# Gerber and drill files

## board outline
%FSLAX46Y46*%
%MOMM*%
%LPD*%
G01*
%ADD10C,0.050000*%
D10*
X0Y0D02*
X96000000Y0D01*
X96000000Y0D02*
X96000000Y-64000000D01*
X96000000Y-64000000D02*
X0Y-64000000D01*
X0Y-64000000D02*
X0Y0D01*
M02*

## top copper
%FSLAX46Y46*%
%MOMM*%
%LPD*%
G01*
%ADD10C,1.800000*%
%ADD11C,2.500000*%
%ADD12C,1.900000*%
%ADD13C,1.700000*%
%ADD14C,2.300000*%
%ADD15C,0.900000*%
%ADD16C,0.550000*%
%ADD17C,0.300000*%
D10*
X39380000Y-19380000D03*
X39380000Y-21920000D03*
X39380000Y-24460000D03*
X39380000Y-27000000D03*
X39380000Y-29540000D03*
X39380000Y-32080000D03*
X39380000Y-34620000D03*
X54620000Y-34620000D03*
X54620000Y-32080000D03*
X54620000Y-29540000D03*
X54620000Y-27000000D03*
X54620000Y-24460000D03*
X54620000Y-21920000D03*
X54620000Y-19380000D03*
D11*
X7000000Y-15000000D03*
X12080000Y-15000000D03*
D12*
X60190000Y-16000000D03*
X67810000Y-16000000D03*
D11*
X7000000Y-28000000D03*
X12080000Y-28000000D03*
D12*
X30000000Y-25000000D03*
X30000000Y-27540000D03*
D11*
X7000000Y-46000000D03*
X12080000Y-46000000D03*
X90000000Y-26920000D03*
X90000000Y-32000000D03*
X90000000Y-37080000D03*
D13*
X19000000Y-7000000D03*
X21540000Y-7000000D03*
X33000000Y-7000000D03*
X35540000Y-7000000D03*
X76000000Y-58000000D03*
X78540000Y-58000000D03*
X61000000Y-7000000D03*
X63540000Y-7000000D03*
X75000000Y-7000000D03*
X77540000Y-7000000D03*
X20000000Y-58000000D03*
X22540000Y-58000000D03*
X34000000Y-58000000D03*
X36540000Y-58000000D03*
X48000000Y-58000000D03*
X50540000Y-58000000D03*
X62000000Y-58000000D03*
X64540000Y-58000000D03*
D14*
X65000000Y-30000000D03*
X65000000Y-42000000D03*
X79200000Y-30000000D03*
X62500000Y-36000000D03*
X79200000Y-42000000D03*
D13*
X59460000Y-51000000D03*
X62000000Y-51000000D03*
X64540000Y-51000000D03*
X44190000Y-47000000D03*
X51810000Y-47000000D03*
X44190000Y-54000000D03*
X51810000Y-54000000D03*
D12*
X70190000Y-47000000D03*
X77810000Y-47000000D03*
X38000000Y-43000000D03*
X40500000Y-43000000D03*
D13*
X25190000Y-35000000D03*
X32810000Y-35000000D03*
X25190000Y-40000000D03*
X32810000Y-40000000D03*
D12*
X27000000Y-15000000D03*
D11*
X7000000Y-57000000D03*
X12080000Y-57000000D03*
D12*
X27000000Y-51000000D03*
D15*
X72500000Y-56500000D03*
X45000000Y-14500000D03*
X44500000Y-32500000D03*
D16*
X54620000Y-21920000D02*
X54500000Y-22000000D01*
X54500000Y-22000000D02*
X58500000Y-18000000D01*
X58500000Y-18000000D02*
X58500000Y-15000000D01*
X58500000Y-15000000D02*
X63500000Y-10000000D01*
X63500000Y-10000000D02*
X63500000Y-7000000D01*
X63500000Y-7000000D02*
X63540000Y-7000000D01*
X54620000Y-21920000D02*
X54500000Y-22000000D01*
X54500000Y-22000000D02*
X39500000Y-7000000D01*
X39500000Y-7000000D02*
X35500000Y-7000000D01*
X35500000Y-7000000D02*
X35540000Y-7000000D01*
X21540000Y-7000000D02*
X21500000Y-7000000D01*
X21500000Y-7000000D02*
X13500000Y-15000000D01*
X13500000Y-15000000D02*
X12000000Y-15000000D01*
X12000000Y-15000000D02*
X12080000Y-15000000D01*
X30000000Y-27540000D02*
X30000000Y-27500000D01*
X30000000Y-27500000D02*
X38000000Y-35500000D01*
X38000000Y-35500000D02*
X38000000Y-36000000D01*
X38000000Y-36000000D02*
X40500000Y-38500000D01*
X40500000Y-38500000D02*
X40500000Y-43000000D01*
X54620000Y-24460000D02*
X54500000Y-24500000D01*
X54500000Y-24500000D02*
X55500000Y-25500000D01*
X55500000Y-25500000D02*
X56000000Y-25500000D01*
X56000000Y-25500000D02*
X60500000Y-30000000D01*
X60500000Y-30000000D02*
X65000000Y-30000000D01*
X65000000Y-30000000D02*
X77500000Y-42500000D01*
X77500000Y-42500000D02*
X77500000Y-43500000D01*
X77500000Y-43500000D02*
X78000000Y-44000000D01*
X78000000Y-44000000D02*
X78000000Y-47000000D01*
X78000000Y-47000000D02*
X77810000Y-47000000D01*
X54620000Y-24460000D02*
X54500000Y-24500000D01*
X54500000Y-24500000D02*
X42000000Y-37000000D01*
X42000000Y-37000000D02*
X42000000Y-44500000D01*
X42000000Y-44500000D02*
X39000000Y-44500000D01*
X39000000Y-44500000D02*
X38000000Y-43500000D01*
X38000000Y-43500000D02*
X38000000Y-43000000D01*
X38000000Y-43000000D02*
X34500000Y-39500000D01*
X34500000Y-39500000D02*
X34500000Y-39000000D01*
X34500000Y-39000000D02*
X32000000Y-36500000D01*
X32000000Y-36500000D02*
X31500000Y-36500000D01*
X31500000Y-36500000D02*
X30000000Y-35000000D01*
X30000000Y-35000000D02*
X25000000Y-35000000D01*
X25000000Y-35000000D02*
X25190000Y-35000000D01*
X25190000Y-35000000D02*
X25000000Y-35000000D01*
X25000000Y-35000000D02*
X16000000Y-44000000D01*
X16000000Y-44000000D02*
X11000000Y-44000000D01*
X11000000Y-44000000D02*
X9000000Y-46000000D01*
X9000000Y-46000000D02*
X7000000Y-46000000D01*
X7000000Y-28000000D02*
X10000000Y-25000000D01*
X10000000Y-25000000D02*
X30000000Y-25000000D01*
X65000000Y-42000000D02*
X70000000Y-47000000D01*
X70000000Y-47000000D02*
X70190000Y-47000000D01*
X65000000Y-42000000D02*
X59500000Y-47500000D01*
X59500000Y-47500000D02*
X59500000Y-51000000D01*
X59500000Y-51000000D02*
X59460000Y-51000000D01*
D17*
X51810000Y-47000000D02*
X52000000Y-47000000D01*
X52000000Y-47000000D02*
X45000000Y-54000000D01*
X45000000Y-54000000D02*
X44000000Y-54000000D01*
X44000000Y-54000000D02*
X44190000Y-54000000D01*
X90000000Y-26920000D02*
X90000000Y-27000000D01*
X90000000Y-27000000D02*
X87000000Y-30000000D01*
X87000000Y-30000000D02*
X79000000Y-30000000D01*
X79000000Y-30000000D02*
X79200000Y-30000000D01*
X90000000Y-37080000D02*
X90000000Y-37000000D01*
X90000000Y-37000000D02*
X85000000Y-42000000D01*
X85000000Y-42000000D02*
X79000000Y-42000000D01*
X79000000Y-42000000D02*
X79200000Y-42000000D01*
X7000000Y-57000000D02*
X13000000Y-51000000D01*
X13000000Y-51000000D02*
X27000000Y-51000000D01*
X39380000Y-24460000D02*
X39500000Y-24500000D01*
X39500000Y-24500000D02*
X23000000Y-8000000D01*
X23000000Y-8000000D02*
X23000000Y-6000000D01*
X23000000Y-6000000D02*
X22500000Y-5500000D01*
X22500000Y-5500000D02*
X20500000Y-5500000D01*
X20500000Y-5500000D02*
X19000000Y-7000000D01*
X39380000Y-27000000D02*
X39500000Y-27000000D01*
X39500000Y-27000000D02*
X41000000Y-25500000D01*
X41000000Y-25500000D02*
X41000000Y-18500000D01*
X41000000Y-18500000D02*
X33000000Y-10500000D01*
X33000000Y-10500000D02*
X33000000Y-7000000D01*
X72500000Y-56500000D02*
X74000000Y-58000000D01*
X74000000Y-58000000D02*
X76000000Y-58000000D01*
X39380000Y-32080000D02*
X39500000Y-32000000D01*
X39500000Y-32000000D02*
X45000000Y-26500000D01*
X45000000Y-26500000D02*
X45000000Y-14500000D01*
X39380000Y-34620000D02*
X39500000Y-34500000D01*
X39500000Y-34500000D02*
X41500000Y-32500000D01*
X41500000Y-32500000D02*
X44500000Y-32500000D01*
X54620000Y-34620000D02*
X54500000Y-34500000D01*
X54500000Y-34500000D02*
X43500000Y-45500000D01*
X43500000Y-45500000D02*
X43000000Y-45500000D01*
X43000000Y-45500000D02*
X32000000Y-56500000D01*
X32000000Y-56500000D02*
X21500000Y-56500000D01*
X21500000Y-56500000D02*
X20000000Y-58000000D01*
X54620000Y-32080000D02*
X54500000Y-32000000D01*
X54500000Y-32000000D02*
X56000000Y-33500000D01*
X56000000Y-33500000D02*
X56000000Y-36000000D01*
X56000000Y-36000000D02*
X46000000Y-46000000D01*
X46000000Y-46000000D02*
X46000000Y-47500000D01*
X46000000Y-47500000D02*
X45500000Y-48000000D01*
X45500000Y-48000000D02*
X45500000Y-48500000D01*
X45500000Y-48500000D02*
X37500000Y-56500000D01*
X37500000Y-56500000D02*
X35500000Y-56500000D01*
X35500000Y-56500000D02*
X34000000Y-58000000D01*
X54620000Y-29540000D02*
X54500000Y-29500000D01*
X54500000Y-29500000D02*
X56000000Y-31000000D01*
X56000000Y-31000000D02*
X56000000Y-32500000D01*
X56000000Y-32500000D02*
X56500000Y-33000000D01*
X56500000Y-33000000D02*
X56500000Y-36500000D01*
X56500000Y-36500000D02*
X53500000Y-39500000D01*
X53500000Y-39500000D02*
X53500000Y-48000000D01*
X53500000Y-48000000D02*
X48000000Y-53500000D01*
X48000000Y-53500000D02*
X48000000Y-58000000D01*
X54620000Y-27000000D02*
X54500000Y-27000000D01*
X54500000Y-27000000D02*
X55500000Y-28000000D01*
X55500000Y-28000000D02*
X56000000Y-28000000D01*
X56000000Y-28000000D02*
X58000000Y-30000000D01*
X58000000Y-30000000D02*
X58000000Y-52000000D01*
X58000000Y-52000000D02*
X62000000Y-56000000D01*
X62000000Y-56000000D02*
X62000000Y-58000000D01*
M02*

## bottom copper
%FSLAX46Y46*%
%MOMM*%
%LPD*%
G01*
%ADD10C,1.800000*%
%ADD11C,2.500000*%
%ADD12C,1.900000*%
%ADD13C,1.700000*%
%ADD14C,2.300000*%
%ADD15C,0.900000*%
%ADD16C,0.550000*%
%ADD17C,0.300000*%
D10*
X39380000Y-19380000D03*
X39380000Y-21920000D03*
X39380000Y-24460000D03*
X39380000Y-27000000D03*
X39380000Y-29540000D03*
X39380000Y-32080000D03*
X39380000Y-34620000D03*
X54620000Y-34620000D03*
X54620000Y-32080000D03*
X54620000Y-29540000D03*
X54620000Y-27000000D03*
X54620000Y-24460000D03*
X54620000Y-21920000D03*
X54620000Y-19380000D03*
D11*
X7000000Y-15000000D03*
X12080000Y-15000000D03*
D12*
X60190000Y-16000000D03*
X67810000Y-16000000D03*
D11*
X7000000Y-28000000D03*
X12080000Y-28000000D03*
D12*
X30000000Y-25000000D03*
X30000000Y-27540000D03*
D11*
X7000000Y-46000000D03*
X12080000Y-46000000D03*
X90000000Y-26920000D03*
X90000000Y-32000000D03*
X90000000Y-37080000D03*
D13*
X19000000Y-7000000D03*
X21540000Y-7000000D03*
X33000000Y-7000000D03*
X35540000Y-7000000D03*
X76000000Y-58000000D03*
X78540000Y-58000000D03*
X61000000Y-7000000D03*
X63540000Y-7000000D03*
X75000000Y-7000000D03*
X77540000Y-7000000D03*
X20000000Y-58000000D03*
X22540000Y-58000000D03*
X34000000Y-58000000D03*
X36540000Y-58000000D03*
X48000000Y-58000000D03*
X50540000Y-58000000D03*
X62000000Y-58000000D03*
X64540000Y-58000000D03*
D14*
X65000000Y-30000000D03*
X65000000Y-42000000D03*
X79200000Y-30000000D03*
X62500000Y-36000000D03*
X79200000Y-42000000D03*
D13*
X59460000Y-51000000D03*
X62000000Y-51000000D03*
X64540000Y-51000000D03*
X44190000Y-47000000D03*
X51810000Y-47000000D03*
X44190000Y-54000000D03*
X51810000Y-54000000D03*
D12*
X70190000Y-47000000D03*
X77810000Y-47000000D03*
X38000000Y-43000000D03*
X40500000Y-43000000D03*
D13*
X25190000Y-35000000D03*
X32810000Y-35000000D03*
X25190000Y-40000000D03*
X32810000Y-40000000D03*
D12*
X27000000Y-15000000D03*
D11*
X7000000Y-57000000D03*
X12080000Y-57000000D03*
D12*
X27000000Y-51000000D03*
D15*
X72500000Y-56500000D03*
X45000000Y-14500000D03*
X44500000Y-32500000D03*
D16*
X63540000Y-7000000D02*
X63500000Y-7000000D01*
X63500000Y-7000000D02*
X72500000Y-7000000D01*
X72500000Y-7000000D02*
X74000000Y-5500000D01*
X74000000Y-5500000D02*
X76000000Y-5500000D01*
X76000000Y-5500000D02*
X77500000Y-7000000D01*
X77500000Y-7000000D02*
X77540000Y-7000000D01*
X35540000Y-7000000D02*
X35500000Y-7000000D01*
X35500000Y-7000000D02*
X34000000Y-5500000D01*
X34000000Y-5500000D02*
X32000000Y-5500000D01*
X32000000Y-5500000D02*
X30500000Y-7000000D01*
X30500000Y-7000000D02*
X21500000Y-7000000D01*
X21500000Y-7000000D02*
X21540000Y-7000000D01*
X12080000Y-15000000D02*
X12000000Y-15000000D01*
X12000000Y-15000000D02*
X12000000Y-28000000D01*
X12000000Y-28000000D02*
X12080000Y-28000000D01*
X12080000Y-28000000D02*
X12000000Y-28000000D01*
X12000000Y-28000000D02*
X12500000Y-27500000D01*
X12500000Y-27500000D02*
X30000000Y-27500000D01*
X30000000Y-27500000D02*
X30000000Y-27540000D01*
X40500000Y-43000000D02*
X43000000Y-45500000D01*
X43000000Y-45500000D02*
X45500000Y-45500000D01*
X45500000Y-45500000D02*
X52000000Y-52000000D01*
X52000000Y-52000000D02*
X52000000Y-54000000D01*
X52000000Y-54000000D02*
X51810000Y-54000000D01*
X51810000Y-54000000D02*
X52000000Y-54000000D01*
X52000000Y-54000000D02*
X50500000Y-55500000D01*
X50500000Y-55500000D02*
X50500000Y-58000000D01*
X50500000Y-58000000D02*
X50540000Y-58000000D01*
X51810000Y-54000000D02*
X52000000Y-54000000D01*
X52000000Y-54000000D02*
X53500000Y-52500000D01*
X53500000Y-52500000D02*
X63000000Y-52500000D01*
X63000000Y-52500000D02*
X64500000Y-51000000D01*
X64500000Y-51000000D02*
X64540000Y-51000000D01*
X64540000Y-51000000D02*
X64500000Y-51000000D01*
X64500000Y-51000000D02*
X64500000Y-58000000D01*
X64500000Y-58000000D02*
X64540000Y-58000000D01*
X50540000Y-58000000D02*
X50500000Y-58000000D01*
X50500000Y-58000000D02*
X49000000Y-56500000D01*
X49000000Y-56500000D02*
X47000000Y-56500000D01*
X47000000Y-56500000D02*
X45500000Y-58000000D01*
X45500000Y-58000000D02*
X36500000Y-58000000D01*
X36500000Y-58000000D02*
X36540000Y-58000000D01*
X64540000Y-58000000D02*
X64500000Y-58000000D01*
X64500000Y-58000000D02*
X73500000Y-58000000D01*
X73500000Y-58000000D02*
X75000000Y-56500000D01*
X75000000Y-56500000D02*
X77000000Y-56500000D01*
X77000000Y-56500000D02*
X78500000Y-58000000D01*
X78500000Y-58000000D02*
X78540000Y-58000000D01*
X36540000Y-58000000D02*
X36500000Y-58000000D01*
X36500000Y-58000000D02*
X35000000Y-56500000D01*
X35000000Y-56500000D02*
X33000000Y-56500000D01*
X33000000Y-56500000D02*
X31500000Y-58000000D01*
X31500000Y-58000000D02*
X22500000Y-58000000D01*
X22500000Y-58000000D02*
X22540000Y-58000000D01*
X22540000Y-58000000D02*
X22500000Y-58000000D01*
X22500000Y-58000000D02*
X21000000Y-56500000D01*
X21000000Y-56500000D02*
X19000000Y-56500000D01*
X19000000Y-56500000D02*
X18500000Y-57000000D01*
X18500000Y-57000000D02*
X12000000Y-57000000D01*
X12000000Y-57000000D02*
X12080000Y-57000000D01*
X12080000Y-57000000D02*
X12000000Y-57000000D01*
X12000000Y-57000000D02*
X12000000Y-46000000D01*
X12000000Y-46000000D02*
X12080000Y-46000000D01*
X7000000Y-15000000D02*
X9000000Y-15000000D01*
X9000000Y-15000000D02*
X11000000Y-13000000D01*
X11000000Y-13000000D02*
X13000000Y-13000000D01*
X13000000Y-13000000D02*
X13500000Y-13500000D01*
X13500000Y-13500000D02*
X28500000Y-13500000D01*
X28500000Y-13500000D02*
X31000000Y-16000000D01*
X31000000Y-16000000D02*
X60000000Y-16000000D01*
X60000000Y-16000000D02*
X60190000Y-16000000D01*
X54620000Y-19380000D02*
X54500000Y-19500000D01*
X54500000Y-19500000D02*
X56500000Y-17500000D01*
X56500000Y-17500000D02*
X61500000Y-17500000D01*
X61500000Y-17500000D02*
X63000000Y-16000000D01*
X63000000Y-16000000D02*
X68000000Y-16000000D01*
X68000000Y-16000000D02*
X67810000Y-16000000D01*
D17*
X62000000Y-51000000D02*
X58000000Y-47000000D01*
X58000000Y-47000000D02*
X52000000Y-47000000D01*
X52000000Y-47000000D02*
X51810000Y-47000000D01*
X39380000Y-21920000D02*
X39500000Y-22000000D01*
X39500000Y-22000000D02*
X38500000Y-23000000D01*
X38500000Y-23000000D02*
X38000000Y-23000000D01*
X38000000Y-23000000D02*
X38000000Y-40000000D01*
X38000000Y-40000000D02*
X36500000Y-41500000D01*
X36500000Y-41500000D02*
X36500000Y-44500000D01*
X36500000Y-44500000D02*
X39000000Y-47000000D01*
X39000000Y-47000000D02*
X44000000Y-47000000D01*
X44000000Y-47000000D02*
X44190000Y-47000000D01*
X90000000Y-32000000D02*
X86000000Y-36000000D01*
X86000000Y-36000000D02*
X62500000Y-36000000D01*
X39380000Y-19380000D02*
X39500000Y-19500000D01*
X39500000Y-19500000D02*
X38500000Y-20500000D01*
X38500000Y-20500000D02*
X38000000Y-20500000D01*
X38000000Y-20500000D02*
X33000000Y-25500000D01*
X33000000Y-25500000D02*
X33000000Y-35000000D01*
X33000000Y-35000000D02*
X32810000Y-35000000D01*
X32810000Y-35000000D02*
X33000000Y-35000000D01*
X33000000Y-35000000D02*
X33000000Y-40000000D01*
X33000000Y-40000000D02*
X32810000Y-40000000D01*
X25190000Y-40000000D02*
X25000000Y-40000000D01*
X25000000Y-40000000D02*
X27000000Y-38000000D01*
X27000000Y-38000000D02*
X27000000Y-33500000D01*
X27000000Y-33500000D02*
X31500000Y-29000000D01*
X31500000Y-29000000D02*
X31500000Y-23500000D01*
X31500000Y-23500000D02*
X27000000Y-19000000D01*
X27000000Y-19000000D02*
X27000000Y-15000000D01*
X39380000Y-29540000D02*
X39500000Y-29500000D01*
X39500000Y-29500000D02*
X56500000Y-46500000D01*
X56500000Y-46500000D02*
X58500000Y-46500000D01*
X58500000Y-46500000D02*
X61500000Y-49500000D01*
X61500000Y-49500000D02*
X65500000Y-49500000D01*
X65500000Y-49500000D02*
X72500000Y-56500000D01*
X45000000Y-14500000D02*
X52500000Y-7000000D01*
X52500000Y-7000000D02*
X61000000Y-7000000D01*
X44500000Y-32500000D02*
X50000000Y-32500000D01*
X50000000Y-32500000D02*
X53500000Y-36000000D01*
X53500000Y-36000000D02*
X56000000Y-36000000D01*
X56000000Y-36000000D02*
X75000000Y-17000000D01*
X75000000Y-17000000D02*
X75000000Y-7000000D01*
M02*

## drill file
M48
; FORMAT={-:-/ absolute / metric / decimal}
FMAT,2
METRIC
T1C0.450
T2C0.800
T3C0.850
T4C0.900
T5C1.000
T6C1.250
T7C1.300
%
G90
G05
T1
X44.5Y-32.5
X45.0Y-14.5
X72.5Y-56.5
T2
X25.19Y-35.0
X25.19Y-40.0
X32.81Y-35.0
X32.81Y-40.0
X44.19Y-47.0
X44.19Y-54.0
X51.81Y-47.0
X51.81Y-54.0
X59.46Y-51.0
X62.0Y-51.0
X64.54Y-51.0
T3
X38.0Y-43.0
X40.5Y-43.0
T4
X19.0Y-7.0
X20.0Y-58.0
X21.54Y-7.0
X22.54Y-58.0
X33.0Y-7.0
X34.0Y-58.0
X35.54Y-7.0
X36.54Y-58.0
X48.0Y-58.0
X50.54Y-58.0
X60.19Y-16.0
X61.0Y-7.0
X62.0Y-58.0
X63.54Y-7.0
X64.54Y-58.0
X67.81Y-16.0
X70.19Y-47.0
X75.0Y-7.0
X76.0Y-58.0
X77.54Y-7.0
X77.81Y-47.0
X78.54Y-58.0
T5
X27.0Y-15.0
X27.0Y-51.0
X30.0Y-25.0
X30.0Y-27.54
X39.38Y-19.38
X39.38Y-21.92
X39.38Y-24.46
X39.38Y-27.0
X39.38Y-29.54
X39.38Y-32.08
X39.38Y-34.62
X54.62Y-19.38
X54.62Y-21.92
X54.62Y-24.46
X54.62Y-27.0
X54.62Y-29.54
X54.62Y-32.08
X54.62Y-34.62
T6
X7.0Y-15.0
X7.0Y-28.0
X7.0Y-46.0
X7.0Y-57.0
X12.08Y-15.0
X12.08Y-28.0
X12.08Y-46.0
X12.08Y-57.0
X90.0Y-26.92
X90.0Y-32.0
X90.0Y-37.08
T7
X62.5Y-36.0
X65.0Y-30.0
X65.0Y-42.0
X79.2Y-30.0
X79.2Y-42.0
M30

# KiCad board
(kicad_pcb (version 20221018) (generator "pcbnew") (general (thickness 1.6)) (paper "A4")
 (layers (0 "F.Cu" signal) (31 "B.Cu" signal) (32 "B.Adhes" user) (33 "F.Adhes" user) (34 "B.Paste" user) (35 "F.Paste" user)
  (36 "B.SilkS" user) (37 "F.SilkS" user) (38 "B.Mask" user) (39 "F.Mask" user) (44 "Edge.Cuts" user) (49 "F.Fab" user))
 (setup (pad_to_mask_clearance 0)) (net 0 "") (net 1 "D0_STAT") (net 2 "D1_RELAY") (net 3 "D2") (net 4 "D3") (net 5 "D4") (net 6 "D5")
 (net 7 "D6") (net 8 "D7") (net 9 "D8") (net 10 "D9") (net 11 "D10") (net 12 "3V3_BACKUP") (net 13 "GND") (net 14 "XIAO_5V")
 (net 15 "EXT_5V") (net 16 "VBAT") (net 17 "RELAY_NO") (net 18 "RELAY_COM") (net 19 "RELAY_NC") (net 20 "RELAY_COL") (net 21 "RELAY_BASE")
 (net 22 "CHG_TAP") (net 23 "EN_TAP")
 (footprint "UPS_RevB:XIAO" (layer "F.Cu") (at 47 27)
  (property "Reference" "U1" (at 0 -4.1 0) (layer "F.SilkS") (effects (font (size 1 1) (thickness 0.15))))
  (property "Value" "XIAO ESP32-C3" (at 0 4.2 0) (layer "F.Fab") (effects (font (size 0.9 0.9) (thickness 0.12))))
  (pad "1" thru_hole circle (at -7.62 -7.62) (size 1.8 1.8) (drill 1) (layers "*.Cu" "*.Mask") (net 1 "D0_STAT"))
  (pad "2" thru_hole circle (at -7.62 -5.08) (size 1.8 1.8) (drill 1) (layers "*.Cu" "*.Mask") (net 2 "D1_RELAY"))
  (pad "3" thru_hole circle (at -7.62 -2.54) (size 1.8 1.8) (drill 1) (layers "*.Cu" "*.Mask") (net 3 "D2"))
  (pad "4" thru_hole circle (at -7.62 0) (size 1.8 1.8) (drill 1) (layers "*.Cu" "*.Mask") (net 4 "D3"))
  (pad "5" thru_hole circle (at -7.62 2.54) (size 1.8 1.8) (drill 1) (layers "*.Cu" "*.Mask") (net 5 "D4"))
  (pad "6" thru_hole circle (at -7.62 5.08) (size 1.8 1.8) (drill 1) (layers "*.Cu" "*.Mask") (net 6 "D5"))
  (pad "7" thru_hole circle (at -7.62 7.62) (size 1.8 1.8) (drill 1) (layers "*.Cu" "*.Mask") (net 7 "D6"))
  (pad "8" thru_hole circle (at 7.62 7.62) (size 1.8 1.8) (drill 1) (layers "*.Cu" "*.Mask") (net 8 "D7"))
  (pad "9" thru_hole circle (at 7.62 5.08) (size 1.8 1.8) (drill 1) (layers "*.Cu" "*.Mask") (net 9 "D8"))
  (pad "10" thru_hole circle (at 7.62 2.54) (size 1.8 1.8) (drill 1) (layers "*.Cu" "*.Mask") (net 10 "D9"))
  (pad "11" thru_hole circle (at 7.62 0) (size 1.8 1.8) (drill 1) (layers "*.Cu" "*.Mask") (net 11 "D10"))
  (pad "12" thru_hole circle (at 7.62 -2.54) (size 1.8 1.8) (drill 1) (layers "*.Cu" "*.Mask") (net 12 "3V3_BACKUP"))
  (pad "13" thru_hole circle (at 7.62 -5.08) (size 1.8 1.8) (drill 1) (layers "*.Cu" "*.Mask") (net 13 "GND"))
  (pad "14" thru_hole circle (at 7.62 -7.62) (size 1.8 1.8) (drill 1) (layers "*.Cu" "*.Mask") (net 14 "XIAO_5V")))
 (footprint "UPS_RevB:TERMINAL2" (layer "F.Cu") (at 7 15)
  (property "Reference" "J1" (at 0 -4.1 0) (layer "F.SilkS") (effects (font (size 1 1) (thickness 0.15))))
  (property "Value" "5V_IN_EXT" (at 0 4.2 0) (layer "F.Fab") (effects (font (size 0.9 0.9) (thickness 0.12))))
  (pad "1" thru_hole circle (at 0 0) (size 2.5 2.5) (drill 1.25) (layers "*.Cu" "*.Mask") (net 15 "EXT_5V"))
  (pad "2" thru_hole circle (at 5.08 0) (size 2.5 2.5) (drill 1.25) (layers "*.Cu" "*.Mask") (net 13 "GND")))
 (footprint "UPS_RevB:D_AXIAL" (layer "F.Cu") (at 64 16)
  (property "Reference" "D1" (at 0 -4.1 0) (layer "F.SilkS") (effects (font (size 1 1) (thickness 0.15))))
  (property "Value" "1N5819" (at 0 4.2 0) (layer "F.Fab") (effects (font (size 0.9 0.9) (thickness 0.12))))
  (pad "1" thru_hole circle (at -3.81 0) (size 1.9 1.9) (drill 0.9) (layers "*.Cu" "*.Mask") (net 15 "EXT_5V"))
  (pad "2" thru_hole circle (at 3.81 0) (size 1.9 1.9) (drill 0.9) (layers "*.Cu" "*.Mask") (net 14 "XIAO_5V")))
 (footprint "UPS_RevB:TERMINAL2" (layer "F.Cu") (at 7 28)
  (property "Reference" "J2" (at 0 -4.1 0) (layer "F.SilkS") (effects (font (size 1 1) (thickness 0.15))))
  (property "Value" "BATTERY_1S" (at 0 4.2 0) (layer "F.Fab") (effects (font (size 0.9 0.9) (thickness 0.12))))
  (pad "1" thru_hole circle (at 0 0) (size 2.5 2.5) (drill 1.25) (layers "*.Cu" "*.Mask") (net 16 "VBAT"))
  (pad "2" thru_hole circle (at 5.08 0) (size 2.5 2.5) (drill 1.25) (layers "*.Cu" "*.Mask") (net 13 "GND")))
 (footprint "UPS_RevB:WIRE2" (layer "F.Cu") (at 30 25)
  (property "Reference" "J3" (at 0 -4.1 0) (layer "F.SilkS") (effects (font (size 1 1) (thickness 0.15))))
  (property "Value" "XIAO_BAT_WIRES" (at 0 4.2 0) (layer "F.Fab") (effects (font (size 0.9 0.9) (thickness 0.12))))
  (pad "1" thru_hole circle (at 0 0) (size 1.9 1.9) (drill 1) (layers "*.Cu" "*.Mask") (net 16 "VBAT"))
  (pad "2" thru_hole circle (at 0 2.54) (size 1.9 1.9) (drill 1) (layers "*.Cu" "*.Mask") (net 13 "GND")))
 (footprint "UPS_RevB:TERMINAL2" (layer "F.Cu") (at 7 46)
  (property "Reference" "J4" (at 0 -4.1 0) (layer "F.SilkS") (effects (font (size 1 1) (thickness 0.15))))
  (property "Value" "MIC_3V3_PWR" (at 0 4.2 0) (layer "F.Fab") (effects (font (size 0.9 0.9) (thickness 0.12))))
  (pad "1" thru_hole circle (at 0 0) (size 2.5 2.5) (drill 1.25) (layers "*.Cu" "*.Mask") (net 12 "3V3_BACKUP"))
  (pad "2" thru_hole circle (at 5.08 0) (size 2.5 2.5) (drill 1.25) (layers "*.Cu" "*.Mask") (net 13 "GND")))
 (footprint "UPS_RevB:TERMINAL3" (layer "F.Cu") (at 90 32)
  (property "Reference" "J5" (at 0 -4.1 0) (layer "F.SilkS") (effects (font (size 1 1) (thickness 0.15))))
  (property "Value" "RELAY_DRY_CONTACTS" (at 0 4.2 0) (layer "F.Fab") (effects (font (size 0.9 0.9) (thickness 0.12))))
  (pad "1" thru_hole circle (at 0 -5.08) (size 2.5 2.5) (drill 1.25) (layers "*.Cu" "*.Mask") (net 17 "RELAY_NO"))
  (pad "2" thru_hole circle (at 0 0) (size 2.5 2.5) (drill 1.25) (layers "*.Cu" "*.Mask") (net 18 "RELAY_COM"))
  (pad "3" thru_hole circle (at 0 5.08) (size 2.5 2.5) (drill 1.25) (layers "*.Cu" "*.Mask") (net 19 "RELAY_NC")))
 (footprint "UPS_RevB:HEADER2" (layer "F.Cu") (at 19 7)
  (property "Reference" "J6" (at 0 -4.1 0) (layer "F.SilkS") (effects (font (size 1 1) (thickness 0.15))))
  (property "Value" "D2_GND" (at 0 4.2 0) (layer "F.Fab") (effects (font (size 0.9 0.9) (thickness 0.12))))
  (pad "1" thru_hole circle (at 0 0) (size 1.7 1.7) (drill 0.9) (layers "*.Cu" "*.Mask") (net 3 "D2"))
  (pad "2" thru_hole circle (at 2.54 0) (size 1.7 1.7) (drill 0.9) (layers "*.Cu" "*.Mask") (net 13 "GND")))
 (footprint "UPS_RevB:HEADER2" (layer "F.Cu") (at 33 7)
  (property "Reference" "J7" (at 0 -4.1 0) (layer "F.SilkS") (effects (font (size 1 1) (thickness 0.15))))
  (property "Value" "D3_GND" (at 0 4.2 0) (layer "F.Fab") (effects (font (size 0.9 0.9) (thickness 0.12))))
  (pad "1" thru_hole circle (at 0 0) (size 1.7 1.7) (drill 0.9) (layers "*.Cu" "*.Mask") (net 4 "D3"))
  (pad "2" thru_hole circle (at 2.54 0) (size 1.7 1.7) (drill 0.9) (layers "*.Cu" "*.Mask") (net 13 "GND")))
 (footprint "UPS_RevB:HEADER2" (layer "F.Cu") (at 76 58)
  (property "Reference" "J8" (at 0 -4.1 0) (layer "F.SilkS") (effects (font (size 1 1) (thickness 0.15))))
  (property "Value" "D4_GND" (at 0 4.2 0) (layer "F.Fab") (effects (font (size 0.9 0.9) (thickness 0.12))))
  (pad "1" thru_hole circle (at 0 0) (size 1.7 1.7) (drill 0.9) (layers "*.Cu" "*.Mask") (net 5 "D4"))
  (pad "2" thru_hole circle (at 2.54 0) (size 1.7 1.7) (drill 0.9) (layers "*.Cu" "*.Mask") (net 13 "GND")))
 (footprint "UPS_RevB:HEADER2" (layer "F.Cu") (at 61 7)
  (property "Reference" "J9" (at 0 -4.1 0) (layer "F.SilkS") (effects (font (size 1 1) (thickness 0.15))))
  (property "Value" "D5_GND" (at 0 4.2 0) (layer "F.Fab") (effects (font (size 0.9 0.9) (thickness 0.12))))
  (pad "1" thru_hole circle (at 0 0) (size 1.7 1.7) (drill 0.9) (layers "*.Cu" "*.Mask") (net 6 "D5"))
  (pad "2" thru_hole circle (at 2.54 0) (size 1.7 1.7) (drill 0.9) (layers "*.Cu" "*.Mask") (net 13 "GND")))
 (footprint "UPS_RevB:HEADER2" (layer "F.Cu") (at 75 7)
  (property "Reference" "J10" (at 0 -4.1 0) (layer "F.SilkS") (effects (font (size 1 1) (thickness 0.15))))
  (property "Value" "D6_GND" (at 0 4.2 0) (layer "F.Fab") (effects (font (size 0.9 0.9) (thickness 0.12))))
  (pad "1" thru_hole circle (at 0 0) (size 1.7 1.7) (drill 0.9) (layers "*.Cu" "*.Mask") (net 7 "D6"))
  (pad "2" thru_hole circle (at 2.54 0) (size 1.7 1.7) (drill 0.9) (layers "*.Cu" "*.Mask") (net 13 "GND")))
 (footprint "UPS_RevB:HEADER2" (layer "F.Cu") (at 20 58)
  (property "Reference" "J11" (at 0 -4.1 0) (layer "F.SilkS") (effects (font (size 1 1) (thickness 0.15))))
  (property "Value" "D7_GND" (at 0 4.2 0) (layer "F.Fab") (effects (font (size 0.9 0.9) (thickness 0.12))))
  (pad "1" thru_hole circle (at 0 0) (size 1.7 1.7) (drill 0.9) (layers "*.Cu" "*.Mask") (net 8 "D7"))
  (pad "2" thru_hole circle (at 2.54 0) (size 1.7 1.7) (drill 0.9) (layers "*.Cu" "*.Mask") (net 13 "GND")))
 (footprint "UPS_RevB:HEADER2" (layer "F.Cu") (at 34 58)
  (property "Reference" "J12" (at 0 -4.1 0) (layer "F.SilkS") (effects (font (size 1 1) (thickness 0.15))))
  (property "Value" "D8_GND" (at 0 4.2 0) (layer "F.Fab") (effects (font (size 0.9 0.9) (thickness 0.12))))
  (pad "1" thru_hole circle (at 0 0) (size 1.7 1.7) (drill 0.9) (layers "*.Cu" "*.Mask") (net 9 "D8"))
  (pad "2" thru_hole circle (at 2.54 0) (size 1.7 1.7) (drill 0.9) (layers "*.Cu" "*.Mask") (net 13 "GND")))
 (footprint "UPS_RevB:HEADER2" (layer "F.Cu") (at 48 58)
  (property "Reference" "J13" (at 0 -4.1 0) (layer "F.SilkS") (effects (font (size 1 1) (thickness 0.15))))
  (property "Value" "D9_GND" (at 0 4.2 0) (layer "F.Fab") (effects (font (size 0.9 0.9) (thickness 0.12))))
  (pad "1" thru_hole circle (at 0 0) (size 1.7 1.7) (drill 0.9) (layers "*.Cu" "*.Mask") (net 10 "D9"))
  (pad "2" thru_hole circle (at 2.54 0) (size 1.7 1.7) (drill 0.9) (layers "*.Cu" "*.Mask") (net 13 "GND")))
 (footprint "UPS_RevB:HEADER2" (layer "F.Cu") (at 62 58)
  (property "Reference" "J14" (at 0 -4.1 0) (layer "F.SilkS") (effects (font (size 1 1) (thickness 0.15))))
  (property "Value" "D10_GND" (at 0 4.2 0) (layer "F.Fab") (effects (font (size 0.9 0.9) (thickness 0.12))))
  (pad "1" thru_hole circle (at 0 0) (size 1.7 1.7) (drill 0.9) (layers "*.Cu" "*.Mask") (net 11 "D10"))
  (pad "2" thru_hole circle (at 2.54 0) (size 1.7 1.7) (drill 0.9) (layers "*.Cu" "*.Mask") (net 13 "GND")))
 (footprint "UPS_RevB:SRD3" (layer "F.Cu") (at 65 30)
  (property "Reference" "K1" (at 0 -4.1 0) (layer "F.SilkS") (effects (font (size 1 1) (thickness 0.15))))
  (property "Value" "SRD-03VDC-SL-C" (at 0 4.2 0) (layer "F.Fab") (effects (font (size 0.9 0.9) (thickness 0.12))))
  (pad "1" thru_hole circle (at 0 0) (size 2.3 2.3) (drill 1.3) (layers "*.Cu" "*.Mask") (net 12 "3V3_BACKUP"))
  (pad "2" thru_hole circle (at 0 12) (size 2.3 2.3) (drill 1.3) (layers "*.Cu" "*.Mask") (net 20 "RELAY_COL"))
  (pad "3" thru_hole circle (at 14.2 0) (size 2.3 2.3) (drill 1.3) (layers "*.Cu" "*.Mask") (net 17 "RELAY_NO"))
  (pad "4" thru_hole circle (at -2.5 6) (size 2.3 2.3) (drill 1.3) (layers "*.Cu" "*.Mask") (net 18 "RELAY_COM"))
  (pad "5" thru_hole circle (at 14.2 12) (size 2.3 2.3) (drill 1.3) (layers "*.Cu" "*.Mask") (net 19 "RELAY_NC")))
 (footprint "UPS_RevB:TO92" (layer "F.Cu") (at 62 51)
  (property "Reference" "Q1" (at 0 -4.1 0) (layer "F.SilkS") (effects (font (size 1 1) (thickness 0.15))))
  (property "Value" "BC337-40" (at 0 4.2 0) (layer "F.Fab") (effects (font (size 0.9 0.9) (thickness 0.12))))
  (pad "1" thru_hole circle (at -2.54 0) (size 1.7 1.7) (drill 0.8) (layers "*.Cu" "*.Mask") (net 20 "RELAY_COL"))
  (pad "2" thru_hole circle (at 0 0) (size 1.7 1.7) (drill 0.8) (layers "*.Cu" "*.Mask") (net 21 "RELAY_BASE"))
  (pad "3" thru_hole circle (at 2.54 0) (size 1.7 1.7) (drill 0.8) (layers "*.Cu" "*.Mask") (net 13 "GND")))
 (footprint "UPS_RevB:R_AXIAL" (layer "F.Cu") (at 48 47)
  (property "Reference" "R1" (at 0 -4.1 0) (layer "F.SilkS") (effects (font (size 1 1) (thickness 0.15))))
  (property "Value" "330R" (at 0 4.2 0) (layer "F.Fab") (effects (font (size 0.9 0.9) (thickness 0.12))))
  (pad "1" thru_hole circle (at -3.81 0) (size 1.7 1.7) (drill 0.8) (layers "*.Cu" "*.Mask") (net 2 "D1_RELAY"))
  (pad "2" thru_hole circle (at 3.81 0) (size 1.7 1.7) (drill 0.8) (layers "*.Cu" "*.Mask") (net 21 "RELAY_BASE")))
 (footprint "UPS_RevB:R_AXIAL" (layer "F.Cu") (at 48 54)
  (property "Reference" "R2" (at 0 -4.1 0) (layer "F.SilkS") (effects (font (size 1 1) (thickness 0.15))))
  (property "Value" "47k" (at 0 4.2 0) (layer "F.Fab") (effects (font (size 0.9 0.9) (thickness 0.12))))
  (pad "1" thru_hole circle (at -3.81 0) (size 1.7 1.7) (drill 0.8) (layers "*.Cu" "*.Mask") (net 21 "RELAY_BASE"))
  (pad "2" thru_hole circle (at 3.81 0) (size 1.7 1.7) (drill 0.8) (layers "*.Cu" "*.Mask") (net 13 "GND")))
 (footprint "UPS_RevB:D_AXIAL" (layer "F.Cu") (at 74 47)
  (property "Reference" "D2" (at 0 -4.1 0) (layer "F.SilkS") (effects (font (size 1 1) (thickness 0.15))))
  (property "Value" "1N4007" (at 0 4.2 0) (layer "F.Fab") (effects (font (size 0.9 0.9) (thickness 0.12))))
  (pad "1" thru_hole circle (at -3.81 0) (size 1.9 1.9) (drill 0.9) (layers "*.Cu" "*.Mask") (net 20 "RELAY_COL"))
  (pad "2" thru_hole circle (at 3.81 0) (size 1.9 1.9) (drill 0.9) (layers "*.Cu" "*.Mask") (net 12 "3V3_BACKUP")))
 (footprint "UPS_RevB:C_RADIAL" (layer "F.Cu") (at 38 43)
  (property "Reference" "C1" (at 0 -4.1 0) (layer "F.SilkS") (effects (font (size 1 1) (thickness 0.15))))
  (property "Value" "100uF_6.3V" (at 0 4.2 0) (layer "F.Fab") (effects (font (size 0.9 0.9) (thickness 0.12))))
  (pad "1" thru_hole circle (at 0 0) (size 1.9 1.9) (drill 0.85) (layers "*.Cu" "*.Mask") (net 12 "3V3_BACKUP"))
  (pad "2" thru_hole circle (at 2.5 0) (size 1.9 1.9) (drill 0.85) (layers "*.Cu" "*.Mask") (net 13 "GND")))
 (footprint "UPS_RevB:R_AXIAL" (layer "F.Cu") (at 29 35)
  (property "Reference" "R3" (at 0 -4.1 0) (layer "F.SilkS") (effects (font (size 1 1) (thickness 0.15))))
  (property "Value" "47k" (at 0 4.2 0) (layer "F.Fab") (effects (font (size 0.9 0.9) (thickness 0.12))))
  (pad "1" thru_hole circle (at -3.81 0) (size 1.7 1.7) (drill 0.8) (layers "*.Cu" "*.Mask") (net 12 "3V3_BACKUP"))
  (pad "2" thru_hole circle (at 3.81 0) (size 1.7 1.7) (drill 0.8) (layers "*.Cu" "*.Mask") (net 1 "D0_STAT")))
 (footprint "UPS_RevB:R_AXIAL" (layer "F.Cu") (at 29 40)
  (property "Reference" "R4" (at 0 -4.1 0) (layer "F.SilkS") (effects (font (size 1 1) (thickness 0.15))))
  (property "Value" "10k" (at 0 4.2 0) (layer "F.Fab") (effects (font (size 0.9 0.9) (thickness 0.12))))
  (pad "1" thru_hole circle (at -3.81 0) (size 1.7 1.7) (drill 0.8) (layers "*.Cu" "*.Mask") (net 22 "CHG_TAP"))
  (pad "2" thru_hole circle (at 3.81 0) (size 1.7 1.7) (drill 0.8) (layers "*.Cu" "*.Mask") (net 1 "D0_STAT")))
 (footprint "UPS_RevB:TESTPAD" (layer "F.Cu") (at 27 15)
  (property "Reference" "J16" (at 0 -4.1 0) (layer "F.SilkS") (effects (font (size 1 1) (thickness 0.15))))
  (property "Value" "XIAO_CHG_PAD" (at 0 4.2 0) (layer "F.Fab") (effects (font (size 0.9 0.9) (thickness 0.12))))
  (pad "1" thru_hole circle (at 0 0) (size 1.9 1.9) (drill 1) (layers "*.Cu" "*.Mask") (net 22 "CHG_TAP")))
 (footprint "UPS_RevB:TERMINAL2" (layer "F.Cu") (at 7 57)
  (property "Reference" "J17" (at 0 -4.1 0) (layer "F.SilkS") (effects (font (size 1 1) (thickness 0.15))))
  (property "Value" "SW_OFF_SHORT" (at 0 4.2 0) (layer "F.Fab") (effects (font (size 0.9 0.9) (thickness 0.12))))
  (pad "1" thru_hole circle (at 0 0) (size 2.5 2.5) (drill 1.25) (layers "*.Cu" "*.Mask") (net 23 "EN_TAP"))
  (pad "2" thru_hole circle (at 5.08 0) (size 2.5 2.5) (drill 1.25) (layers "*.Cu" "*.Mask") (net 13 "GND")))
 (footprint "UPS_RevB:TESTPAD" (layer "F.Cu") (at 27 51)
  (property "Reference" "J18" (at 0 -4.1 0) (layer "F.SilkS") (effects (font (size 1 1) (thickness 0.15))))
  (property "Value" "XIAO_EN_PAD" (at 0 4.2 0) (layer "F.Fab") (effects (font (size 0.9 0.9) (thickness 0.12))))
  (pad "1" thru_hole circle (at 0 0) (size 1.9 1.9) (drill 1) (layers "*.Cu" "*.Mask") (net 23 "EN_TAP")))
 (gr_line (start 0 0) (end 96 0) (stroke (width 0.05) (type default)) (layer "Edge.Cuts"))
 (gr_line (start 96 0) (end 96 64) (stroke (width 0.05) (type default)) (layer "Edge.Cuts"))
 (gr_line (start 96 64) (end 0 64) (stroke (width 0.05) (type default)) (layer "Edge.Cuts"))
 (gr_line (start 0 64) (end 0 0) (stroke (width 0.05) (type default)) (layer "Edge.Cuts"))
 (segment (start 54.62 21.92) (end 54.5 22) (width 0.55) (layer "F.Cu") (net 13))
 (segment (start 54.5 22) (end 58.5 18) (width 0.55) (layer "F.Cu") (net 13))
 (segment (start 58.5 18) (end 58.5 15) (width 0.55) (layer "F.Cu") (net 13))
 (segment (start 58.5 15) (end 63.5 10) (width 0.55) (layer "F.Cu") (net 13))
 (segment (start 63.5 10) (end 63.5 7) (width 0.55) (layer "F.Cu") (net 13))
 (segment (start 63.5 7) (end 63.54 7) (width 0.55) (layer "F.Cu") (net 13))
 (segment (start 63.54 7) (end 63.5 7) (width 0.55) (layer "B.Cu") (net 13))
 (segment (start 63.5 7) (end 72.5 7) (width 0.55) (layer "B.Cu") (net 13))
 (segment (start 72.5 7) (end 74 5.5) (width 0.55) (layer "B.Cu") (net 13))
 (segment (start 74 5.5) (end 76 5.5) (width 0.55) (layer "B.Cu") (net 13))
 (segment (start 76 5.5) (end 77.5 7) (width 0.55) (layer "B.Cu") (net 13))
 (segment (start 77.5 7) (end 77.54 7) (width 0.55) (layer "B.Cu") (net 13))
 (segment (start 54.62 21.92) (end 54.5 22) (width 0.55) (layer "F.Cu") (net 13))
 (segment (start 54.5 22) (end 39.5 7) (width 0.55) (layer "F.Cu") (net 13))
 (segment (start 39.5 7) (end 35.5 7) (width 0.55) (layer "F.Cu") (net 13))
 (segment (start 35.5 7) (end 35.54 7) (width 0.55) (layer "F.Cu") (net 13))
 (segment (start 35.54 7) (end 35.5 7) (width 0.55) (layer "B.Cu") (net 13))
 (segment (start 35.5 7) (end 34 5.5) (width 0.55) (layer "B.Cu") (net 13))
 (segment (start 34 5.5) (end 32 5.5) (width 0.55) (layer "B.Cu") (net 13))
 (segment (start 32 5.5) (end 30.5 7) (width 0.55) (layer "B.Cu") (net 13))
 (segment (start 30.5 7) (end 21.5 7) (width 0.55) (layer "B.Cu") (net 13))
 (segment (start 21.5 7) (end 21.54 7) (width 0.55) (layer "B.Cu") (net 13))
 (segment (start 21.54 7) (end 21.5 7) (width 0.55) (layer "F.Cu") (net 13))
 (segment (start 21.5 7) (end 13.5 15) (width 0.55) (layer "F.Cu") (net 13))
 (segment (start 13.5 15) (end 12 15) (width 0.55) (layer "F.Cu") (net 13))
 (segment (start 12 15) (end 12.08 15) (width 0.55) (layer "F.Cu") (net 13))
 (segment (start 12.08 15) (end 12 15) (width 0.55) (layer "B.Cu") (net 13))
 (segment (start 12 15) (end 12 28) (width 0.55) (layer "B.Cu") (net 13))
 (segment (start 12 28) (end 12.08 28) (width 0.55) (layer "B.Cu") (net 13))
 (segment (start 12.08 28) (end 12 28) (width 0.55) (layer "B.Cu") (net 13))
 (segment (start 12 28) (end 12.5 27.5) (width 0.55) (layer "B.Cu") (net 13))
 (segment (start 12.5 27.5) (end 30 27.5) (width 0.55) (layer "B.Cu") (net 13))
 (segment (start 30 27.5) (end 30 27.54) (width 0.55) (layer "B.Cu") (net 13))
 (segment (start 30 27.54) (end 30 27.5) (width 0.55) (layer "F.Cu") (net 13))
 (segment (start 30 27.5) (end 38 35.5) (width 0.55) (layer "F.Cu") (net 13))
 (segment (start 38 35.5) (end 38 36) (width 0.55) (layer "F.Cu") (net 13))
 (segment (start 38 36) (end 40.5 38.5) (width 0.55) (layer "F.Cu") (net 13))
 (segment (start 40.5 38.5) (end 40.5 43) (width 0.55) (layer "F.Cu") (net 13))
 (segment (start 40.5 43) (end 43 45.5) (width 0.55) (layer "B.Cu") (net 13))
 (segment (start 43 45.5) (end 45.5 45.5) (width 0.55) (layer "B.Cu") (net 13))
 (segment (start 45.5 45.5) (end 52 52) (width 0.55) (layer "B.Cu") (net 13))
 (segment (start 52 52) (end 52 54) (width 0.55) (layer "B.Cu") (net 13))
 (segment (start 52 54) (end 51.81 54) (width 0.55) (layer "B.Cu") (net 13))
 (segment (start 51.81 54) (end 52 54) (width 0.55) (layer "B.Cu") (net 13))
 (segment (start 52 54) (end 50.5 55.5) (width 0.55) (layer "B.Cu") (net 13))
 (segment (start 50.5 55.5) (end 50.5 58) (width 0.55) (layer "B.Cu") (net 13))
 (segment (start 50.5 58) (end 50.54 58) (width 0.55) (layer "B.Cu") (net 13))
 (segment (start 51.81 54) (end 52 54) (width 0.55) (layer "B.Cu") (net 13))
 (segment (start 52 54) (end 53.5 52.5) (width 0.55) (layer "B.Cu") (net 13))
 (segment (start 53.5 52.5) (end 63 52.5) (width 0.55) (layer "B.Cu") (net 13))
 (segment (start 63 52.5) (end 64.5 51) (width 0.55) (layer "B.Cu") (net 13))
 (segment (start 64.5 51) (end 64.54 51) (width 0.55) (layer "B.Cu") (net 13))
 (segment (start 64.54 51) (end 64.5 51) (width 0.55) (layer "B.Cu") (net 13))
 (segment (start 64.5 51) (end 64.5 58) (width 0.55) (layer "B.Cu") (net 13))
 (segment (start 64.5 58) (end 64.54 58) (width 0.55) (layer "B.Cu") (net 13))
 (segment (start 50.54 58) (end 50.5 58) (width 0.55) (layer "B.Cu") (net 13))
 (segment (start 50.5 58) (end 49 56.5) (width 0.55) (layer "B.Cu") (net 13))
 (segment (start 49 56.5) (end 47 56.5) (width 0.55) (layer "B.Cu") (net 13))
 (segment (start 47 56.5) (end 45.5 58) (width 0.55) (layer "B.Cu") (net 13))
 (segment (start 45.5 58) (end 36.5 58) (width 0.55) (layer "B.Cu") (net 13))
 (segment (start 36.5 58) (end 36.54 58) (width 0.55) (layer "B.Cu") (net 13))
 (segment (start 64.54 58) (end 64.5 58) (width 0.55) (layer "B.Cu") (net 13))
 (segment (start 64.5 58) (end 73.5 58) (width 0.55) (layer "B.Cu") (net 13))
 (segment (start 73.5 58) (end 75 56.5) (width 0.55) (layer "B.Cu") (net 13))
 (segment (start 75 56.5) (end 77 56.5) (width 0.55) (layer "B.Cu") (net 13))
 (segment (start 77 56.5) (end 78.5 58) (width 0.55) (layer "B.Cu") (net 13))
 (segment (start 78.5 58) (end 78.54 58) (width 0.55) (layer "B.Cu") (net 13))
 (segment (start 36.54 58) (end 36.5 58) (width 0.55) (layer "B.Cu") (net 13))
 (segment (start 36.5 58) (end 35 56.5) (width 0.55) (layer "B.Cu") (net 13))
 (segment (start 35 56.5) (end 33 56.5) (width 0.55) (layer "B.Cu") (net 13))
 (segment (start 33 56.5) (end 31.5 58) (width 0.55) (layer "B.Cu") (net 13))
 (segment (start 31.5 58) (end 22.5 58) (width 0.55) (layer "B.Cu") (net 13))
 (segment (start 22.5 58) (end 22.54 58) (width 0.55) (layer "B.Cu") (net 13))
 (segment (start 22.54 58) (end 22.5 58) (width 0.55) (layer "B.Cu") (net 13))
 (segment (start 22.5 58) (end 21 56.5) (width 0.55) (layer "B.Cu") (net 13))
 (segment (start 21 56.5) (end 19 56.5) (width 0.55) (layer "B.Cu") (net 13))
 (segment (start 19 56.5) (end 18.5 57) (width 0.55) (layer "B.Cu") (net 13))
 (segment (start 18.5 57) (end 12 57) (width 0.55) (layer "B.Cu") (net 13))
 (segment (start 12 57) (end 12.08 57) (width 0.55) (layer "B.Cu") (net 13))
 (segment (start 12.08 57) (end 12 57) (width 0.55) (layer "B.Cu") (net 13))
 (segment (start 12 57) (end 12 46) (width 0.55) (layer "B.Cu") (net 13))
 (segment (start 12 46) (end 12.08 46) (width 0.55) (layer "B.Cu") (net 13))
 (segment (start 54.62 24.46) (end 54.5 24.5) (width 0.55) (layer "F.Cu") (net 12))
 (segment (start 54.5 24.5) (end 55.5 25.5) (width 0.55) (layer "F.Cu") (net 12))
 (segment (start 55.5 25.5) (end 56 25.5) (width 0.55) (layer "F.Cu") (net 12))
 (segment (start 56 25.5) (end 60.5 30) (width 0.55) (layer "F.Cu") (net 12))
 (segment (start 60.5 30) (end 65 30) (width 0.55) (layer "F.Cu") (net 12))
 (segment (start 65 30) (end 77.5 42.5) (width 0.55) (layer "F.Cu") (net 12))
 (segment (start 77.5 42.5) (end 77.5 43.5) (width 0.55) (layer "F.Cu") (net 12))
 (segment (start 77.5 43.5) (end 78 44) (width 0.55) (layer "F.Cu") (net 12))
 (segment (start 78 44) (end 78 47) (width 0.55) (layer "F.Cu") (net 12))
 (segment (start 78 47) (end 77.81 47) (width 0.55) (layer "F.Cu") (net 12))
 (segment (start 54.62 24.46) (end 54.5 24.5) (width 0.55) (layer "F.Cu") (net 12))
 (segment (start 54.5 24.5) (end 42 37) (width 0.55) (layer "F.Cu") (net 12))
 (segment (start 42 37) (end 42 44.5) (width 0.55) (layer "F.Cu") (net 12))
 (segment (start 42 44.5) (end 39 44.5) (width 0.55) (layer "F.Cu") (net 12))
 (segment (start 39 44.5) (end 38 43.5) (width 0.55) (layer "F.Cu") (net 12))
 (segment (start 38 43.5) (end 38 43) (width 0.55) (layer "F.Cu") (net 12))
 (segment (start 38 43) (end 34.5 39.5) (width 0.55) (layer "F.Cu") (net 12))
 (segment (start 34.5 39.5) (end 34.5 39) (width 0.55) (layer "F.Cu") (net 12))
 (segment (start 34.5 39) (end 32 36.5) (width 0.55) (layer "F.Cu") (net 12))
 (segment (start 32 36.5) (end 31.5 36.5) (width 0.55) (layer "F.Cu") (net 12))
 (segment (start 31.5 36.5) (end 30 35) (width 0.55) (layer "F.Cu") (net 12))
 (segment (start 30 35) (end 25 35) (width 0.55) (layer "F.Cu") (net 12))
 (segment (start 25 35) (end 25.19 35) (width 0.55) (layer "F.Cu") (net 12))
 (segment (start 25.19 35) (end 25 35) (width 0.55) (layer "F.Cu") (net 12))
 (segment (start 25 35) (end 16 44) (width 0.55) (layer "F.Cu") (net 12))
 (segment (start 16 44) (end 11 44) (width 0.55) (layer "F.Cu") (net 12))
 (segment (start 11 44) (end 9 46) (width 0.55) (layer "F.Cu") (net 12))
 (segment (start 9 46) (end 7 46) (width 0.55) (layer "F.Cu") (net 12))
 (segment (start 7 28) (end 10 25) (width 0.55) (layer "F.Cu") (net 16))
 (segment (start 10 25) (end 30 25) (width 0.55) (layer "F.Cu") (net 16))
 (segment (start 7 15) (end 9 15) (width 0.55) (layer "B.Cu") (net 15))
 (segment (start 9 15) (end 11 13) (width 0.55) (layer "B.Cu") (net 15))
 (segment (start 11 13) (end 13 13) (width 0.55) (layer "B.Cu") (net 15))
 (segment (start 13 13) (end 13.5 13.5) (width 0.55) (layer "B.Cu") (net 15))
 (segment (start 13.5 13.5) (end 28.5 13.5) (width 0.55) (layer "B.Cu") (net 15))
 (segment (start 28.5 13.5) (end 31 16) (width 0.55) (layer "B.Cu") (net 15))
 (segment (start 31 16) (end 60 16) (width 0.55) (layer "B.Cu") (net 15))
 (segment (start 60 16) (end 60.19 16) (width 0.55) (layer "B.Cu") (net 15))
 (segment (start 54.62 19.38) (end 54.5 19.5) (width 0.55) (layer "B.Cu") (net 14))
 (segment (start 54.5 19.5) (end 56.5 17.5) (width 0.55) (layer "B.Cu") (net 14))
 (segment (start 56.5 17.5) (end 61.5 17.5) (width 0.55) (layer "B.Cu") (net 14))
 (segment (start 61.5 17.5) (end 63 16) (width 0.55) (layer "B.Cu") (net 14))
 (segment (start 63 16) (end 68 16) (width 0.55) (layer "B.Cu") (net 14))
 (segment (start 68 16) (end 67.81 16) (width 0.55) (layer "B.Cu") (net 14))
 (segment (start 65 42) (end 70 47) (width 0.55) (layer "F.Cu") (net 20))
 (segment (start 70 47) (end 70.19 47) (width 0.55) (layer "F.Cu") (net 20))
 (segment (start 65 42) (end 59.5 47.5) (width 0.55) (layer "F.Cu") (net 20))
 (segment (start 59.5 47.5) (end 59.5 51) (width 0.55) (layer "F.Cu") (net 20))
 (segment (start 59.5 51) (end 59.46 51) (width 0.55) (layer "F.Cu") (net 20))
 (segment (start 62 51) (end 58 47) (width 0.3) (layer "B.Cu") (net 21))
 (segment (start 58 47) (end 52 47) (width 0.3) (layer "B.Cu") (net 21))
 (segment (start 52 47) (end 51.81 47) (width 0.3) (layer "B.Cu") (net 21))
 (segment (start 51.81 47) (end 52 47) (width 0.3) (layer "F.Cu") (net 21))
 (segment (start 52 47) (end 45 54) (width 0.3) (layer "F.Cu") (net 21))
 (segment (start 45 54) (end 44 54) (width 0.3) (layer "F.Cu") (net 21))
 (segment (start 44 54) (end 44.19 54) (width 0.3) (layer "F.Cu") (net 21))
 (segment (start 39.38 21.92) (end 39.5 22) (width 0.3) (layer "B.Cu") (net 2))
 (segment (start 39.5 22) (end 38.5 23) (width 0.3) (layer "B.Cu") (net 2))
 (segment (start 38.5 23) (end 38 23) (width 0.3) (layer "B.Cu") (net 2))
 (segment (start 38 23) (end 38 40) (width 0.3) (layer "B.Cu") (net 2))
 (segment (start 38 40) (end 36.5 41.5) (width 0.3) (layer "B.Cu") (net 2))
 (segment (start 36.5 41.5) (end 36.5 44.5) (width 0.3) (layer "B.Cu") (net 2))
 (segment (start 36.5 44.5) (end 39 47) (width 0.3) (layer "B.Cu") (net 2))
 (segment (start 39 47) (end 44 47) (width 0.3) (layer "B.Cu") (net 2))
 (segment (start 44 47) (end 44.19 47) (width 0.3) (layer "B.Cu") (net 2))
 (segment (start 90 26.92) (end 90 27) (width 0.3) (layer "F.Cu") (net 17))
 (segment (start 90 27) (end 87 30) (width 0.3) (layer "F.Cu") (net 17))
 (segment (start 87 30) (end 79 30) (width 0.3) (layer "F.Cu") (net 17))
 (segment (start 79 30) (end 79.2 30) (width 0.3) (layer "F.Cu") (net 17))
 (segment (start 90 32) (end 86 36) (width 0.3) (layer "B.Cu") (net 18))
 (segment (start 86 36) (end 62.5 36) (width 0.3) (layer "B.Cu") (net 18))
 (segment (start 90 37.08) (end 90 37) (width 0.3) (layer "F.Cu") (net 19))
 (segment (start 90 37) (end 85 42) (width 0.3) (layer "F.Cu") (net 19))
 (segment (start 85 42) (end 79 42) (width 0.3) (layer "F.Cu") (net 19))
 (segment (start 79 42) (end 79.2 42) (width 0.3) (layer "F.Cu") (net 19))
 (segment (start 39.38 19.38) (end 39.5 19.5) (width 0.3) (layer "B.Cu") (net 1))
 (segment (start 39.5 19.5) (end 38.5 20.5) (width 0.3) (layer "B.Cu") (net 1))
 (segment (start 38.5 20.5) (end 38 20.5) (width 0.3) (layer "B.Cu") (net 1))
 (segment (start 38 20.5) (end 33 25.5) (width 0.3) (layer "B.Cu") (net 1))
 (segment (start 33 25.5) (end 33 35) (width 0.3) (layer "B.Cu") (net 1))
 (segment (start 33 35) (end 32.81 35) (width 0.3) (layer "B.Cu") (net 1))
 (segment (start 32.81 35) (end 33 35) (width 0.3) (layer "B.Cu") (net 1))
 (segment (start 33 35) (end 33 40) (width 0.3) (layer "B.Cu") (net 1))
 (segment (start 33 40) (end 32.81 40) (width 0.3) (layer "B.Cu") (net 1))
 (segment (start 25.19 40) (end 25 40) (width 0.3) (layer "B.Cu") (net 22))
 (segment (start 25 40) (end 27 38) (width 0.3) (layer "B.Cu") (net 22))
 (segment (start 27 38) (end 27 33.5) (width 0.3) (layer "B.Cu") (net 22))
 (segment (start 27 33.5) (end 31.5 29) (width 0.3) (layer "B.Cu") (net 22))
 (segment (start 31.5 29) (end 31.5 23.5) (width 0.3) (layer "B.Cu") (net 22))
 (segment (start 31.5 23.5) (end 27 19) (width 0.3) (layer "B.Cu") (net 22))
 (segment (start 27 19) (end 27 15) (width 0.3) (layer "B.Cu") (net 22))
 (segment (start 7 57) (end 13 51) (width 0.3) (layer "F.Cu") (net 23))
 (segment (start 13 51) (end 27 51) (width 0.3) (layer "F.Cu") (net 23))
 (segment (start 39.38 24.46) (end 39.5 24.5) (width 0.3) (layer "F.Cu") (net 3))
 (segment (start 39.5 24.5) (end 23 8) (width 0.3) (layer "F.Cu") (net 3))
 (segment (start 23 8) (end 23 6) (width 0.3) (layer "F.Cu") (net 3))
 (segment (start 23 6) (end 22.5 5.5) (width 0.3) (layer "F.Cu") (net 3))
 (segment (start 22.5 5.5) (end 20.5 5.5) (width 0.3) (layer "F.Cu") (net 3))
 (segment (start 20.5 5.5) (end 19 7) (width 0.3) (layer "F.Cu") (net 3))
 (segment (start 39.38 27) (end 39.5 27) (width 0.3) (layer "F.Cu") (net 4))
 (segment (start 39.5 27) (end 41 25.5) (width 0.3) (layer "F.Cu") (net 4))
 (segment (start 41 25.5) (end 41 18.5) (width 0.3) (layer "F.Cu") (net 4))
 (segment (start 41 18.5) (end 33 10.5) (width 0.3) (layer "F.Cu") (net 4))
 (segment (start 33 10.5) (end 33 7) (width 0.3) (layer "F.Cu") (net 4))
 (segment (start 39.38 29.54) (end 39.5 29.5) (width 0.3) (layer "B.Cu") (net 5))
 (segment (start 39.5 29.5) (end 56.5 46.5) (width 0.3) (layer "B.Cu") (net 5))
 (segment (start 56.5 46.5) (end 58.5 46.5) (width 0.3) (layer "B.Cu") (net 5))
 (segment (start 58.5 46.5) (end 61.5 49.5) (width 0.3) (layer "B.Cu") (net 5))
 (segment (start 61.5 49.5) (end 65.5 49.5) (width 0.3) (layer "B.Cu") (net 5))
 (segment (start 65.5 49.5) (end 72.5 56.5) (width 0.3) (layer "B.Cu") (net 5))
 (segment (start 72.5 56.5) (end 74 58) (width 0.3) (layer "F.Cu") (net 5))
 (segment (start 74 58) (end 76 58) (width 0.3) (layer "F.Cu") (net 5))
 (segment (start 39.38 32.08) (end 39.5 32) (width 0.3) (layer "F.Cu") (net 6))
 (segment (start 39.5 32) (end 45 26.5) (width 0.3) (layer "F.Cu") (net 6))
 (segment (start 45 26.5) (end 45 14.5) (width 0.3) (layer "F.Cu") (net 6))
 (segment (start 45 14.5) (end 52.5 7) (width 0.3) (layer "B.Cu") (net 6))
 (segment (start 52.5 7) (end 61 7) (width 0.3) (layer "B.Cu") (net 6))
 (segment (start 39.38 34.62) (end 39.5 34.5) (width 0.3) (layer "F.Cu") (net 7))
 (segment (start 39.5 34.5) (end 41.5 32.5) (width 0.3) (layer "F.Cu") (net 7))
 (segment (start 41.5 32.5) (end 44.5 32.5) (width 0.3) (layer "F.Cu") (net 7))
 (segment (start 44.5 32.5) (end 50 32.5) (width 0.3) (layer "B.Cu") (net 7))
 (segment (start 50 32.5) (end 53.5 36) (width 0.3) (layer "B.Cu") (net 7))
 (segment (start 53.5 36) (end 56 36) (width 0.3) (layer "B.Cu") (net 7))
 (segment (start 56 36) (end 75 17) (width 0.3) (layer "B.Cu") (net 7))
 (segment (start 75 17) (end 75 7) (width 0.3) (layer "B.Cu") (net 7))
 (segment (start 54.62 34.62) (end 54.5 34.5) (width 0.3) (layer "F.Cu") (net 8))
 (segment (start 54.5 34.5) (end 43.5 45.5) (width 0.3) (layer "F.Cu") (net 8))
 (segment (start 43.5 45.5) (end 43 45.5) (width 0.3) (layer "F.Cu") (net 8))
 (segment (start 43 45.5) (end 32 56.5) (width 0.3) (layer "F.Cu") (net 8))
 (segment (start 32 56.5) (end 21.5 56.5) (width 0.3) (layer "F.Cu") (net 8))
 (segment (start 21.5 56.5) (end 20 58) (width 0.3) (layer "F.Cu") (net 8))
 (segment (start 54.62 32.08) (end 54.5 32) (width 0.3) (layer "F.Cu") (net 9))
 (segment (start 54.5 32) (end 56 33.5) (width 0.3) (layer "F.Cu") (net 9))
 (segment (start 56 33.5) (end 56 36) (width 0.3) (layer "F.Cu") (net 9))
 (segment (start 56 36) (end 46 46) (width 0.3) (layer "F.Cu") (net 9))
 (segment (start 46 46) (end 46 47.5) (width 0.3) (layer "F.Cu") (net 9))
 (segment (start 46 47.5) (end 45.5 48) (width 0.3) (layer "F.Cu") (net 9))
 (segment (start 45.5 48) (end 45.5 48.5) (width 0.3) (layer "F.Cu") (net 9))
 (segment (start 45.5 48.5) (end 37.5 56.5) (width 0.3) (layer "F.Cu") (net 9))
 (segment (start 37.5 56.5) (end 35.5 56.5) (width 0.3) (layer "F.Cu") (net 9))
 (segment (start 35.5 56.5) (end 34 58) (width 0.3) (layer "F.Cu") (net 9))
 (segment (start 54.62 29.54) (end 54.5 29.5) (width 0.3) (layer "F.Cu") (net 10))
 (segment (start 54.5 29.5) (end 56 31) (width 0.3) (layer "F.Cu") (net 10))
 (segment (start 56 31) (end 56 32.5) (width 0.3) (layer "F.Cu") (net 10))
 (segment (start 56 32.5) (end 56.5 33) (width 0.3) (layer "F.Cu") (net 10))
 (segment (start 56.5 33) (end 56.5 36.5) (width 0.3) (layer "F.Cu") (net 10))
 (segment (start 56.5 36.5) (end 53.5 39.5) (width 0.3) (layer "F.Cu") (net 10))
 (segment (start 53.5 39.5) (end 53.5 48) (width 0.3) (layer "F.Cu") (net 10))
 (segment (start 53.5 48) (end 48 53.5) (width 0.3) (layer "F.Cu") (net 10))
 (segment (start 48 53.5) (end 48 58) (width 0.3) (layer "F.Cu") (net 10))
 (segment (start 54.62 27) (end 54.5 27) (width 0.3) (layer "F.Cu") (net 11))
 (segment (start 54.5 27) (end 55.5 28) (width 0.3) (layer "F.Cu") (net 11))
 (segment (start 55.5 28) (end 56 28) (width 0.3) (layer "F.Cu") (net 11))
 (segment (start 56 28) (end 58 30) (width 0.3) (layer "F.Cu") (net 11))
 (segment (start 58 30) (end 58 52) (width 0.3) (layer "F.Cu") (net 11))
 (segment (start 58 52) (end 62 56) (width 0.3) (layer "F.Cu") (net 11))
 (segment (start 62 56) (end 62 58) (width 0.3) (layer "F.Cu") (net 11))
 (via (at 72.5 56.5) (size 0.9) (drill 0.45) (layers "F.Cu" "B.Cu") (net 5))
 (via (at 45 14.5) (size 0.9) (drill 0.45) (layers "F.Cu" "B.Cu") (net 6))
 (via (at 44.5 32.5) (size 0.9) (drill 0.45) (layers "F.Cu" "B.Cu") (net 7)))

